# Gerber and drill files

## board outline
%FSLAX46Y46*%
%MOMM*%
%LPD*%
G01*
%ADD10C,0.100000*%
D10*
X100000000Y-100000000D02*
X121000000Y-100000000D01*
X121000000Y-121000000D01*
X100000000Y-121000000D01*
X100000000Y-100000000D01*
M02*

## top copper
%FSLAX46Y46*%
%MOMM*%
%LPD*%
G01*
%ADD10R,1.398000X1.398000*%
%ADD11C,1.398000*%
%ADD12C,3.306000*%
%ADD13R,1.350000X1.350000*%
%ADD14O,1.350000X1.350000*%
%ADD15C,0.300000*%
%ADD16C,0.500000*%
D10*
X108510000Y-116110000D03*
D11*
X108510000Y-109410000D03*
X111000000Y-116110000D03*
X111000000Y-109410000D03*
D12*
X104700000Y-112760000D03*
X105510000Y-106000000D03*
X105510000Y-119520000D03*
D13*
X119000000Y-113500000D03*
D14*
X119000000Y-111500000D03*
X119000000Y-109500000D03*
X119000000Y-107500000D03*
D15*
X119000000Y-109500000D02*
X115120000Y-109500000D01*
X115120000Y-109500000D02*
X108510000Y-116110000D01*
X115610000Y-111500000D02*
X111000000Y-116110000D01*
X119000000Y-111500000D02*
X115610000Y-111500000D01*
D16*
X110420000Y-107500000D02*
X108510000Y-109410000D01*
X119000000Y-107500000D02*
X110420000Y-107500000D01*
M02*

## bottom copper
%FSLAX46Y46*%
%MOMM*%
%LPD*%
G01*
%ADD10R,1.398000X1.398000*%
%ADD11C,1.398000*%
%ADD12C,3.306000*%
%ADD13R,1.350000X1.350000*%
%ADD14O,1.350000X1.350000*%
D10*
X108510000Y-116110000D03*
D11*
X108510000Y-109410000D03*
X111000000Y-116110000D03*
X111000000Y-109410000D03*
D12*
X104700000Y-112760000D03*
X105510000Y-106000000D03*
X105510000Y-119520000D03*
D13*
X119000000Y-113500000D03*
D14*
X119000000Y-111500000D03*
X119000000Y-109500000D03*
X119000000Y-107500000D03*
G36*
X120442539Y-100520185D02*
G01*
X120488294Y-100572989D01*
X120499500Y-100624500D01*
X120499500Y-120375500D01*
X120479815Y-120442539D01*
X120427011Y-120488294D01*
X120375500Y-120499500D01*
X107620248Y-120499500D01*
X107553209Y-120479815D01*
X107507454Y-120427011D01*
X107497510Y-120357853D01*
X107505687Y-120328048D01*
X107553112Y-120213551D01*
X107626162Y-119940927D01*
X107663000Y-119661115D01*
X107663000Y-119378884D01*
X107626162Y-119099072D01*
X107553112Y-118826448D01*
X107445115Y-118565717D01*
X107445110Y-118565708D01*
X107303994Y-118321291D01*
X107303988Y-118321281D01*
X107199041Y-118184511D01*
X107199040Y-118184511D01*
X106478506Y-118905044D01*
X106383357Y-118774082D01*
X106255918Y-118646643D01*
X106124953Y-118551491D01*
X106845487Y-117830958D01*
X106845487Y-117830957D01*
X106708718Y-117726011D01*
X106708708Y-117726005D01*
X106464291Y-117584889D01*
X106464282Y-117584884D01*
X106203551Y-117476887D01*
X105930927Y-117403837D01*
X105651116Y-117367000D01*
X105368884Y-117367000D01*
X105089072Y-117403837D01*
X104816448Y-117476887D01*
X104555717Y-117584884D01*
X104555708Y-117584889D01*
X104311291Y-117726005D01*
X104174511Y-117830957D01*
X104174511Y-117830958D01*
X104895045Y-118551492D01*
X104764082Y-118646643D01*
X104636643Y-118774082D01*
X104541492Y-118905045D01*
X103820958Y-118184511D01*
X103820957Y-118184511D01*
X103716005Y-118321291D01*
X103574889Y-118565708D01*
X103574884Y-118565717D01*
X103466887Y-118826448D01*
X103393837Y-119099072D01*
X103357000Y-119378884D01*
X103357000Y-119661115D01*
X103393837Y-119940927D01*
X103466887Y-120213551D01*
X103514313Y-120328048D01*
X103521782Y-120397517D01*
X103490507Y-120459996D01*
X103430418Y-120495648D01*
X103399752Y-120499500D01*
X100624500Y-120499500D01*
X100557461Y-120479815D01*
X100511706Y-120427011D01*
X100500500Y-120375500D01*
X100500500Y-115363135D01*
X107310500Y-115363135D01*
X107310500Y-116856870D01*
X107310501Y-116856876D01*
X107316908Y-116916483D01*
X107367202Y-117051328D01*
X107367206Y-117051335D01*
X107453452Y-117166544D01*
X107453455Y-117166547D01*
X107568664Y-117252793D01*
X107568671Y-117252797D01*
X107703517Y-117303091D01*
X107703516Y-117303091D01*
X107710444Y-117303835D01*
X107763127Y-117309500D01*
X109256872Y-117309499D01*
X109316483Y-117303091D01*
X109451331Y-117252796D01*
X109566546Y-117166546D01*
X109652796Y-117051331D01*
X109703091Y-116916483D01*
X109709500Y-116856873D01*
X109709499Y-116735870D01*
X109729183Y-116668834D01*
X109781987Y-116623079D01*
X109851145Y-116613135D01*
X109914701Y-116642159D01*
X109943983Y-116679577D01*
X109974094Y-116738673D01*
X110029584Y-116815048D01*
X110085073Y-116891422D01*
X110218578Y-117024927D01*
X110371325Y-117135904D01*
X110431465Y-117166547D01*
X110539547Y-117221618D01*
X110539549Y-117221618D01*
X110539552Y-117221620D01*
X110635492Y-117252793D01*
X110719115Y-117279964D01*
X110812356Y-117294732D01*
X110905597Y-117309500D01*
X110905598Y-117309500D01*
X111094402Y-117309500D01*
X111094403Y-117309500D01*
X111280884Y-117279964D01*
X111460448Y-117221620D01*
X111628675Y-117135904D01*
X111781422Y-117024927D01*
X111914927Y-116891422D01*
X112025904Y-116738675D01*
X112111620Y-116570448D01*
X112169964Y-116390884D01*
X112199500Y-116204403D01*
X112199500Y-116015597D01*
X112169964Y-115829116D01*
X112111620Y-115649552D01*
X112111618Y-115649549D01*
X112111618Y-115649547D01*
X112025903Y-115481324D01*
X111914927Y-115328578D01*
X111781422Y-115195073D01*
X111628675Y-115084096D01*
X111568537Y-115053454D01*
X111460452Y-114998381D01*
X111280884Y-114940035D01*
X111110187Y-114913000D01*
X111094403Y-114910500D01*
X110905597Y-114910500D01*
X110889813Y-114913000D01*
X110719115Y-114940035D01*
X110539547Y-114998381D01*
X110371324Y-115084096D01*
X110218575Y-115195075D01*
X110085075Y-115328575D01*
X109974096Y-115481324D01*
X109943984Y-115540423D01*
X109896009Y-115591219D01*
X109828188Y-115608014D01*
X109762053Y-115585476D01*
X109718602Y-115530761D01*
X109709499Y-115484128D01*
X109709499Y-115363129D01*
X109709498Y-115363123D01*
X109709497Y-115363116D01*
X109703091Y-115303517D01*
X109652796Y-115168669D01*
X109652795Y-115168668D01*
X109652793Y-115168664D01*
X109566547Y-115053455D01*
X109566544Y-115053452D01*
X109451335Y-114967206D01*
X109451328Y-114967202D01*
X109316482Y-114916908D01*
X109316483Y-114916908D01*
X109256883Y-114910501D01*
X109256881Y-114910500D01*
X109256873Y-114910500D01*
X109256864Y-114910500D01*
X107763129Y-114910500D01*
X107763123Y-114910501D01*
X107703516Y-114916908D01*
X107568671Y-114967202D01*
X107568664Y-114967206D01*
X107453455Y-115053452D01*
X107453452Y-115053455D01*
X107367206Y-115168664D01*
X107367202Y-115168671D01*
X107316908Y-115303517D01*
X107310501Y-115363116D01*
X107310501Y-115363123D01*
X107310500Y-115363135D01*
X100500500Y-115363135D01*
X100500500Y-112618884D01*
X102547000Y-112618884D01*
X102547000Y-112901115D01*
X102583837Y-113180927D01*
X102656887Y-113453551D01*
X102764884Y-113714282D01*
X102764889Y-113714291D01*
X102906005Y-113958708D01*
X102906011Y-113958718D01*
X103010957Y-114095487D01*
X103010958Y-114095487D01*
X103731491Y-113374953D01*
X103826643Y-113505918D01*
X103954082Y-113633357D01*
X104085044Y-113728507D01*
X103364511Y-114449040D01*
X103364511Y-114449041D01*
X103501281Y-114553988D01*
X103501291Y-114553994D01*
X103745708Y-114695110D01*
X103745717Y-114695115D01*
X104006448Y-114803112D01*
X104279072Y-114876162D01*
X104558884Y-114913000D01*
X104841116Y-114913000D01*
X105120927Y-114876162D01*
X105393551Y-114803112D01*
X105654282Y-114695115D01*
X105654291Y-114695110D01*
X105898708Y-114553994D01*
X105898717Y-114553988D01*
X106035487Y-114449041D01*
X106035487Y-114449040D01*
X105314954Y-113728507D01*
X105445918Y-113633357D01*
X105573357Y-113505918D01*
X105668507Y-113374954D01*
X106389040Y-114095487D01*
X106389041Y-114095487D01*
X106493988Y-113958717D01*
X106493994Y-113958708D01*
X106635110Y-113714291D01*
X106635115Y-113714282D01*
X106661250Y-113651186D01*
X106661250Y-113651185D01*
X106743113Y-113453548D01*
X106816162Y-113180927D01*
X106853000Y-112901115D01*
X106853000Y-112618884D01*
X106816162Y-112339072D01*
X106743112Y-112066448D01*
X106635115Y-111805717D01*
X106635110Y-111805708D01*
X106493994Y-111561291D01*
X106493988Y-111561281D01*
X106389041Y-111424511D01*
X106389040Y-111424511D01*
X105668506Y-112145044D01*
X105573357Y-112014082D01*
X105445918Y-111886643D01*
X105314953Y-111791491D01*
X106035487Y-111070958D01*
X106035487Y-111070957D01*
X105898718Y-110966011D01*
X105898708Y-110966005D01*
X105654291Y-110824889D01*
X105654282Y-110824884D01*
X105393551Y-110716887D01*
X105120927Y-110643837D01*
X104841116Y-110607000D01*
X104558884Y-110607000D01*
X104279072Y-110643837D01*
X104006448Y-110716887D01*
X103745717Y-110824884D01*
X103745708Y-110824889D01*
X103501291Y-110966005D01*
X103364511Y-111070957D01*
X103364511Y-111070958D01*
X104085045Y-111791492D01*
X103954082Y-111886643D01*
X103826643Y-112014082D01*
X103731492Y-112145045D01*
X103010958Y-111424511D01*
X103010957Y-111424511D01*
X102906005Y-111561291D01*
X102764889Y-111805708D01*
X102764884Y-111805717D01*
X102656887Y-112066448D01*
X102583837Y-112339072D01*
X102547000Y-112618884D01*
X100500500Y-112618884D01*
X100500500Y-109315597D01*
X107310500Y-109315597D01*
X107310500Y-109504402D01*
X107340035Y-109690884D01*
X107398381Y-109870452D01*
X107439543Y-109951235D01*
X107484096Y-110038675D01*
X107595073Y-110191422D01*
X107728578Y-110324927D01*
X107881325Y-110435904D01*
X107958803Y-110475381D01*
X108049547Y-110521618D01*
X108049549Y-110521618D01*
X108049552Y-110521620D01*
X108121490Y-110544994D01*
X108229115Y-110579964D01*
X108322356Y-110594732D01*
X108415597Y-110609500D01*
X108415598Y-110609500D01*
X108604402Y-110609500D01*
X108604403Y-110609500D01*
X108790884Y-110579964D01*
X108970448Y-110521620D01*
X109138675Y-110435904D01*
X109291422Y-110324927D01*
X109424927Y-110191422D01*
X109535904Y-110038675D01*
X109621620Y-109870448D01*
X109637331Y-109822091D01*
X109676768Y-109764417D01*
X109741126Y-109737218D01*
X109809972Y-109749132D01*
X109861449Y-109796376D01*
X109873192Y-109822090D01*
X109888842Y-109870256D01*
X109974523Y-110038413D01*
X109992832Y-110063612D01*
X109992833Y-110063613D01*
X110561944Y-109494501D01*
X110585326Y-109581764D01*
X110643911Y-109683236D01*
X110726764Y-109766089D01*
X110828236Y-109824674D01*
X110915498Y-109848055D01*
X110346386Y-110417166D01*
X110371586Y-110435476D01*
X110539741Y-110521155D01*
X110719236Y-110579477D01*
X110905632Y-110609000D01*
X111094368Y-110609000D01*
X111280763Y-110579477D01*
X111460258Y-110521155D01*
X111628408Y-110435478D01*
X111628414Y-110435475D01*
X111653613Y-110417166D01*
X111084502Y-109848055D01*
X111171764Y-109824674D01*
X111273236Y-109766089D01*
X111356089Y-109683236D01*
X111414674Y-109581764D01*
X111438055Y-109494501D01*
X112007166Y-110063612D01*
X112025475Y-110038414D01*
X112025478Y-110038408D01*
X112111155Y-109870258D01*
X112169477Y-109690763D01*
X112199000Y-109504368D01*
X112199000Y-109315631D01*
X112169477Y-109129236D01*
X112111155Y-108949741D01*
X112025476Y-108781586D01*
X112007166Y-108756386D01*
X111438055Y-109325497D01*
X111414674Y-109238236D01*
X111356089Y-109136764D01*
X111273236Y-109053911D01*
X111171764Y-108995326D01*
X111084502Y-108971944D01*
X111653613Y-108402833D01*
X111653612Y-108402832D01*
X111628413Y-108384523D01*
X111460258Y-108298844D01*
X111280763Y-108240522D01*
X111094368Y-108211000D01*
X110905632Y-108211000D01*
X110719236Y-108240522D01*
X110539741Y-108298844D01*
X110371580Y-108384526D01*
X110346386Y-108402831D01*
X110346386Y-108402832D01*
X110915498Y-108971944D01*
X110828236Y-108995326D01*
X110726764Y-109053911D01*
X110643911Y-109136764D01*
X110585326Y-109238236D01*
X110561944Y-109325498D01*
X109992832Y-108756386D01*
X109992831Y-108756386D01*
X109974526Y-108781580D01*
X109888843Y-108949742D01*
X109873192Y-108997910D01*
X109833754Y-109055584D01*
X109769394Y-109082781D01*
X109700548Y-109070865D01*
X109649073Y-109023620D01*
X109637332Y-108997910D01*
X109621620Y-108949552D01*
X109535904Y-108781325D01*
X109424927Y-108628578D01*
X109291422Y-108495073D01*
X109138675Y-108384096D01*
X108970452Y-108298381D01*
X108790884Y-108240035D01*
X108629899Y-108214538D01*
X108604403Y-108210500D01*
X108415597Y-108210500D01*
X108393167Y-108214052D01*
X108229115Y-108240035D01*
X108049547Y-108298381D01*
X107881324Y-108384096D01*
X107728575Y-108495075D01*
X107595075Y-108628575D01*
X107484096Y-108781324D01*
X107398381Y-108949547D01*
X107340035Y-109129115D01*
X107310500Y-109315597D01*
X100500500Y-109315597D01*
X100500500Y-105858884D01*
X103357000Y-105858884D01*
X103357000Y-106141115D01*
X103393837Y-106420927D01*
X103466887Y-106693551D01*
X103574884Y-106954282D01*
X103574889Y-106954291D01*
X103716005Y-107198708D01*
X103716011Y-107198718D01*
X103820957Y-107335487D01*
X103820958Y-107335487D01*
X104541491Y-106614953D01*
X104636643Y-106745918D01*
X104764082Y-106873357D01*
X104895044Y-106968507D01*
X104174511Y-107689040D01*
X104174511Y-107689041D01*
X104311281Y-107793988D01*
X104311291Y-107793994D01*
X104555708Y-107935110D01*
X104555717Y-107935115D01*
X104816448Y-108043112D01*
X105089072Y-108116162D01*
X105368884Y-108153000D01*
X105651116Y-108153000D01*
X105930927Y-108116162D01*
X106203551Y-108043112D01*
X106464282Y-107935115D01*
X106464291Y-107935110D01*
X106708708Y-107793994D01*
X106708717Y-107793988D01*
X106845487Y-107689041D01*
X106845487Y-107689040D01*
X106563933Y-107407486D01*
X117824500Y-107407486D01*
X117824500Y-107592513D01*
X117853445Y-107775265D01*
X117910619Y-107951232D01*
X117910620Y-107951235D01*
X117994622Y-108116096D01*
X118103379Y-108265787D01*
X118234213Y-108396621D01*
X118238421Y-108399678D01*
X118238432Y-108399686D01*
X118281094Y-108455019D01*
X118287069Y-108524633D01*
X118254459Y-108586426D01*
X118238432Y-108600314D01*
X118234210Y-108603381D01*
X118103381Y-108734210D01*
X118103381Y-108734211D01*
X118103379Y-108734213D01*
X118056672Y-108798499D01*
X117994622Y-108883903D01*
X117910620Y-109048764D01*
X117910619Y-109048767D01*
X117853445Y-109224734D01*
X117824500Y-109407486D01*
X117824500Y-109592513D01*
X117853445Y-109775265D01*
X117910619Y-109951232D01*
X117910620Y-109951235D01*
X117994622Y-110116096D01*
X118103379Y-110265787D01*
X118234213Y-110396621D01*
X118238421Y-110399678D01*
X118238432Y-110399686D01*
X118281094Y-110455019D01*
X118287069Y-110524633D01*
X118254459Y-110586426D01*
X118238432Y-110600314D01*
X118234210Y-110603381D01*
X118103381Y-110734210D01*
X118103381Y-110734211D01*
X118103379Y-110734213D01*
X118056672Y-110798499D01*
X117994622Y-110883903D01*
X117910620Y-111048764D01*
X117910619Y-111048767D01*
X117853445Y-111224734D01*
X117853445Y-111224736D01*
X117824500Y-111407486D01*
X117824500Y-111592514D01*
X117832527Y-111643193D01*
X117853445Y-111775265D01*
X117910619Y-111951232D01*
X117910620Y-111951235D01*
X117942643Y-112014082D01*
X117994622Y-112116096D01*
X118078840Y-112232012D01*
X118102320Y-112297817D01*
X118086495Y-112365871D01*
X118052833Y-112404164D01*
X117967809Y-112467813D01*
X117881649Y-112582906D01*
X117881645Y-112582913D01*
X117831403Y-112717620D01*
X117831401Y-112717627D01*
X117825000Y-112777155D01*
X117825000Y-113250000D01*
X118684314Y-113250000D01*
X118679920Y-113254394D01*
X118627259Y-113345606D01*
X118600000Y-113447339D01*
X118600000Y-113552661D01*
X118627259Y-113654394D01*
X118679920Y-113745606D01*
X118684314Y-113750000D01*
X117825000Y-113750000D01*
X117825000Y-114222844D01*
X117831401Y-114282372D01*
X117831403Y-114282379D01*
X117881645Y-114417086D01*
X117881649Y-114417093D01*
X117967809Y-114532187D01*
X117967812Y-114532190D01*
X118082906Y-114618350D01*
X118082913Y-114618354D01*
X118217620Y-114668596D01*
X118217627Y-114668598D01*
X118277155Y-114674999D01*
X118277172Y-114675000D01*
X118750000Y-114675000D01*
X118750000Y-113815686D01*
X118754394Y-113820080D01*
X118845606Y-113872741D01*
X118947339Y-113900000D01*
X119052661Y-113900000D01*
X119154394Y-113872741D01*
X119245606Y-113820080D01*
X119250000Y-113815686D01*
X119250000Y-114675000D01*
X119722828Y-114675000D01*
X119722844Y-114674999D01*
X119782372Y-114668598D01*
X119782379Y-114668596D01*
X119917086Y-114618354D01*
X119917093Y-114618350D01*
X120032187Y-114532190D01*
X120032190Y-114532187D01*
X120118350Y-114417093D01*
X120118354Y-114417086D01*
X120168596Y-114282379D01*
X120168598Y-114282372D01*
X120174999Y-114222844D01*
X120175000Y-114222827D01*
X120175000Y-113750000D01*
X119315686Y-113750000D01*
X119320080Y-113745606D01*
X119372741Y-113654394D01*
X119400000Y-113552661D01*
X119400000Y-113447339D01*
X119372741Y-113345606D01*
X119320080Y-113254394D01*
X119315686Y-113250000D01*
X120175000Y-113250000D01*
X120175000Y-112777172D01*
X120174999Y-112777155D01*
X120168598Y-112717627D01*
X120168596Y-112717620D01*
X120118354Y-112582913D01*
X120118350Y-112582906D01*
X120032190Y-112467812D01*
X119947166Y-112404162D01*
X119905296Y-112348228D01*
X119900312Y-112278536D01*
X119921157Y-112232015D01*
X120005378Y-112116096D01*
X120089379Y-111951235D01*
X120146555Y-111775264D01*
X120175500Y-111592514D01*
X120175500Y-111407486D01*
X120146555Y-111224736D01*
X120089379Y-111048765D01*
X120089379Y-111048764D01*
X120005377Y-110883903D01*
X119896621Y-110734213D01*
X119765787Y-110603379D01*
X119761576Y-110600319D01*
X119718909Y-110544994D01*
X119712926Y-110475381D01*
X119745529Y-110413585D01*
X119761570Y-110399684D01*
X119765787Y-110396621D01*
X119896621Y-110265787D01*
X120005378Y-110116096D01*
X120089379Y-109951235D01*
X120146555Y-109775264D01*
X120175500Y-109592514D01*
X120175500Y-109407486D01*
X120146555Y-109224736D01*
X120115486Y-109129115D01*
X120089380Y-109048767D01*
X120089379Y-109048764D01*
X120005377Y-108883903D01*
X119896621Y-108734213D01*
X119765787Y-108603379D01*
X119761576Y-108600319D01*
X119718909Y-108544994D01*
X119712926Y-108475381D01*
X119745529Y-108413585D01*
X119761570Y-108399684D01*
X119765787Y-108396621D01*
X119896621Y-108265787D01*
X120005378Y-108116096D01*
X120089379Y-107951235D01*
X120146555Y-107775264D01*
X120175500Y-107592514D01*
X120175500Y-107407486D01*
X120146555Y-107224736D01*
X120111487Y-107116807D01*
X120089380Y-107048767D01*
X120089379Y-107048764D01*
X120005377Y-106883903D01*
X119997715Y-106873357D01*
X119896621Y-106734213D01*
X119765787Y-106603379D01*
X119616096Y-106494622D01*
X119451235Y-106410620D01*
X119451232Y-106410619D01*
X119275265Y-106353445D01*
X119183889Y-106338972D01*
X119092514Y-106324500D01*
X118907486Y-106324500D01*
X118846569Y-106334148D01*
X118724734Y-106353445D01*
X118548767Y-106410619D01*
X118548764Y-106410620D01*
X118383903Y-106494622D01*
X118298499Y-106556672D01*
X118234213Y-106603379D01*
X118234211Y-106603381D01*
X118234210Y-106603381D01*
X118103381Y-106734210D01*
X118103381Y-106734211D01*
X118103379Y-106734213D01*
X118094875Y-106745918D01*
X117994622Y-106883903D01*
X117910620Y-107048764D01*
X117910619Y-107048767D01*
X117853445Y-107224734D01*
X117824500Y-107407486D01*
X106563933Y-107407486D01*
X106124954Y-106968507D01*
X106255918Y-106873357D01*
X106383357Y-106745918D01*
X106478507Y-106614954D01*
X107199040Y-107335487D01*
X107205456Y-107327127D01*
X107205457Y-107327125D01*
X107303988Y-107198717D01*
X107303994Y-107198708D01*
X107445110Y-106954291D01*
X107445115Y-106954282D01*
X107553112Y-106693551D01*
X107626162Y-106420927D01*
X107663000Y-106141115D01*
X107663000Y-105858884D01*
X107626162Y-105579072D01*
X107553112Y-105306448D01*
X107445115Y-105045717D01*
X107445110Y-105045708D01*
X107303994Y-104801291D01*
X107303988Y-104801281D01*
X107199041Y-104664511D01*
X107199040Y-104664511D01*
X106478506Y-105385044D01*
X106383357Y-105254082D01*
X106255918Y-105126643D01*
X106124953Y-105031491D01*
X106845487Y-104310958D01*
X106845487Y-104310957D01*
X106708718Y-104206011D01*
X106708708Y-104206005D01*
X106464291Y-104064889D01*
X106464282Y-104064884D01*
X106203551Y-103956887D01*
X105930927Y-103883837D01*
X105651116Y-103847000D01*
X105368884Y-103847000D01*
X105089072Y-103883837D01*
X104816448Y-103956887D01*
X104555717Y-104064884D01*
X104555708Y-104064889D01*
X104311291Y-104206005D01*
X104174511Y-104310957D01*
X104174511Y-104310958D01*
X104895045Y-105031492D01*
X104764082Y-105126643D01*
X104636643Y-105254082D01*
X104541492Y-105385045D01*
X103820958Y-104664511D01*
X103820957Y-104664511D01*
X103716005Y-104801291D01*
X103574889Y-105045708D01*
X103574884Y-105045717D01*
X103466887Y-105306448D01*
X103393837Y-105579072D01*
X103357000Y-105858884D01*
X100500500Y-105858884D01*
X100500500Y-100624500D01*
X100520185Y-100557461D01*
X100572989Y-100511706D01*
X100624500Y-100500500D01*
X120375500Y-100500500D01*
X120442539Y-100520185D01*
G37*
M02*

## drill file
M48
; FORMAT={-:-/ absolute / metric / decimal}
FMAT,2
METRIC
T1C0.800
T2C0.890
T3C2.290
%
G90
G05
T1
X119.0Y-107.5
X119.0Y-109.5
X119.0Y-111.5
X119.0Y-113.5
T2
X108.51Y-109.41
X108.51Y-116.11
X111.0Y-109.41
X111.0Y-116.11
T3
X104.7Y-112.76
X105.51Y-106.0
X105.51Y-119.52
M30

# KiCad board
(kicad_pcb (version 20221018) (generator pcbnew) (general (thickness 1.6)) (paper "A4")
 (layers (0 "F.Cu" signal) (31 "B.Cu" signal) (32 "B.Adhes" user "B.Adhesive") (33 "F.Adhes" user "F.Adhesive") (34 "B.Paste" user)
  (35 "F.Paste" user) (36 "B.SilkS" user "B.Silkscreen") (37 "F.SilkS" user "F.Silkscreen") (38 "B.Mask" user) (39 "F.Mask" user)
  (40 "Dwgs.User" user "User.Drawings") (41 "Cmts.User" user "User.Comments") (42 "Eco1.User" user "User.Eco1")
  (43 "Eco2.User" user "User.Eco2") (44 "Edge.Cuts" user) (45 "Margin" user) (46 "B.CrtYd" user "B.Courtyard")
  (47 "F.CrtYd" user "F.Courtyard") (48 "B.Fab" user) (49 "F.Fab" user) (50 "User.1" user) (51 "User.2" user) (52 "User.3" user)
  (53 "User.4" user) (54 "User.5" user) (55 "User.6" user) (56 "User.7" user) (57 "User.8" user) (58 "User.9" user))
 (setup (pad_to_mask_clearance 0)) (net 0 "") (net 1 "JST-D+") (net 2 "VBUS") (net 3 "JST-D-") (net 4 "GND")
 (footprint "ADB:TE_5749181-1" (layer "F.Cu") (at 108.51 112.76 90)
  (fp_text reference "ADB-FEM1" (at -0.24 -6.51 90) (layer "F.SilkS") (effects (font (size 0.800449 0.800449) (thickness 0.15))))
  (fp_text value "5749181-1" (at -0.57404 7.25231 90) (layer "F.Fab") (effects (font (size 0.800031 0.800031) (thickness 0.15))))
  (pad "1" thru_hole rect (at -3.35 0 90) (size 1.398 1.398) (drill 0.89) (layers "*.Cu" "*.Mask") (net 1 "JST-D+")
   (solder_mask_margin 0.102))
  (pad "2" thru_hole circle (at 3.35 0 90) (size 1.398 1.398) (drill 0.89) (layers "*.Cu" "*.Mask") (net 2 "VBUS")
   (solder_mask_margin 0.102))
  (pad "3" thru_hole circle (at -3.35 2.49 90) (size 1.398 1.398) (drill 0.89) (layers "*.Cu" "*.Mask") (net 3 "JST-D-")
   (solder_mask_margin 0.102))
  (pad "4" thru_hole circle (at 3.35 2.49 90) (size 1.398 1.398) (drill 0.89) (layers "*.Cu" "*.Mask") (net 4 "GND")
   (solder_mask_margin 0.102))
  (pad "5" thru_hole circle (at 0 -3.81 90) (size 3.306 3.306) (drill 2.29) (layers "*.Cu" "*.Mask") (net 4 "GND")
   (solder_mask_margin 0.102))
  (pad "6" thru_hole circle (at 6.76 -3 90) (size 3.306 3.306) (drill 2.29) (layers "*.Cu" "*.Mask") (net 4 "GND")
   (solder_mask_margin 0.102))
  (pad "7" thru_hole circle (at -6.76 -3 90) (size 3.306 3.306) (drill 2.29) (layers "*.Cu" "*.Mask") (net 4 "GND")
   (solder_mask_margin 0.102)))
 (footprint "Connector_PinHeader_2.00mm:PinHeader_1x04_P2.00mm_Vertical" (layer "F.Cu") (at 119 113.5 180)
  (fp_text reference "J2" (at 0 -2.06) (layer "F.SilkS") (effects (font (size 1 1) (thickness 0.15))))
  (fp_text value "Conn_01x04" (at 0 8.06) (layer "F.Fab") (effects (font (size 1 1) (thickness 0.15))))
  (pad "1" thru_hole rect (at 0 0 180) (size 1.35 1.35) (drill 0.8) (layers "*.Cu" "*.Mask") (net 4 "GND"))
  (pad "2" thru_hole oval (at 0 2 180) (size 1.35 1.35) (drill 0.8) (layers "*.Cu" "*.Mask") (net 3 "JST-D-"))
  (pad "3" thru_hole oval (at 0 4 180) (size 1.35 1.35) (drill 0.8) (layers "*.Cu" "*.Mask") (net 1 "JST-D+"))
  (pad "4" thru_hole oval (at 0 6 180) (size 1.35 1.35) (drill 0.8) (layers "*.Cu" "*.Mask") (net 2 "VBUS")))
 (gr_rect locked (start 100 100) (end 121 121) (stroke (width 0.1) (type default)) (fill none) (layer "Edge.Cuts"))
 (segment (start 119 109.5) (end 115.12 109.5) (width 0.3) (layer "F.Cu") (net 1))
 (segment (start 115.12 109.5) (end 108.51 116.11) (width 0.3) (layer "F.Cu") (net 1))
 (segment (start 115.61 111.5) (end 111 116.11) (width 0.3) (layer "F.Cu") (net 3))
 (segment (start 119 111.5) (end 115.61 111.5) (width 0.3) (layer "F.Cu") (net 3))
 (segment (start 110.42 107.5) (end 108.51 109.41) (width 0.5) (layer "F.Cu") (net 2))
 (segment (start 119 107.5) (end 110.42 107.5) (width 0.5) (layer "F.Cu") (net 2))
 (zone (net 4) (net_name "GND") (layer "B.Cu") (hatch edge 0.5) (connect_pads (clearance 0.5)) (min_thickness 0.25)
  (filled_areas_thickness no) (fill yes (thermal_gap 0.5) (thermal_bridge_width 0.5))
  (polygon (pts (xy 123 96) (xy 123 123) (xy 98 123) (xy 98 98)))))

